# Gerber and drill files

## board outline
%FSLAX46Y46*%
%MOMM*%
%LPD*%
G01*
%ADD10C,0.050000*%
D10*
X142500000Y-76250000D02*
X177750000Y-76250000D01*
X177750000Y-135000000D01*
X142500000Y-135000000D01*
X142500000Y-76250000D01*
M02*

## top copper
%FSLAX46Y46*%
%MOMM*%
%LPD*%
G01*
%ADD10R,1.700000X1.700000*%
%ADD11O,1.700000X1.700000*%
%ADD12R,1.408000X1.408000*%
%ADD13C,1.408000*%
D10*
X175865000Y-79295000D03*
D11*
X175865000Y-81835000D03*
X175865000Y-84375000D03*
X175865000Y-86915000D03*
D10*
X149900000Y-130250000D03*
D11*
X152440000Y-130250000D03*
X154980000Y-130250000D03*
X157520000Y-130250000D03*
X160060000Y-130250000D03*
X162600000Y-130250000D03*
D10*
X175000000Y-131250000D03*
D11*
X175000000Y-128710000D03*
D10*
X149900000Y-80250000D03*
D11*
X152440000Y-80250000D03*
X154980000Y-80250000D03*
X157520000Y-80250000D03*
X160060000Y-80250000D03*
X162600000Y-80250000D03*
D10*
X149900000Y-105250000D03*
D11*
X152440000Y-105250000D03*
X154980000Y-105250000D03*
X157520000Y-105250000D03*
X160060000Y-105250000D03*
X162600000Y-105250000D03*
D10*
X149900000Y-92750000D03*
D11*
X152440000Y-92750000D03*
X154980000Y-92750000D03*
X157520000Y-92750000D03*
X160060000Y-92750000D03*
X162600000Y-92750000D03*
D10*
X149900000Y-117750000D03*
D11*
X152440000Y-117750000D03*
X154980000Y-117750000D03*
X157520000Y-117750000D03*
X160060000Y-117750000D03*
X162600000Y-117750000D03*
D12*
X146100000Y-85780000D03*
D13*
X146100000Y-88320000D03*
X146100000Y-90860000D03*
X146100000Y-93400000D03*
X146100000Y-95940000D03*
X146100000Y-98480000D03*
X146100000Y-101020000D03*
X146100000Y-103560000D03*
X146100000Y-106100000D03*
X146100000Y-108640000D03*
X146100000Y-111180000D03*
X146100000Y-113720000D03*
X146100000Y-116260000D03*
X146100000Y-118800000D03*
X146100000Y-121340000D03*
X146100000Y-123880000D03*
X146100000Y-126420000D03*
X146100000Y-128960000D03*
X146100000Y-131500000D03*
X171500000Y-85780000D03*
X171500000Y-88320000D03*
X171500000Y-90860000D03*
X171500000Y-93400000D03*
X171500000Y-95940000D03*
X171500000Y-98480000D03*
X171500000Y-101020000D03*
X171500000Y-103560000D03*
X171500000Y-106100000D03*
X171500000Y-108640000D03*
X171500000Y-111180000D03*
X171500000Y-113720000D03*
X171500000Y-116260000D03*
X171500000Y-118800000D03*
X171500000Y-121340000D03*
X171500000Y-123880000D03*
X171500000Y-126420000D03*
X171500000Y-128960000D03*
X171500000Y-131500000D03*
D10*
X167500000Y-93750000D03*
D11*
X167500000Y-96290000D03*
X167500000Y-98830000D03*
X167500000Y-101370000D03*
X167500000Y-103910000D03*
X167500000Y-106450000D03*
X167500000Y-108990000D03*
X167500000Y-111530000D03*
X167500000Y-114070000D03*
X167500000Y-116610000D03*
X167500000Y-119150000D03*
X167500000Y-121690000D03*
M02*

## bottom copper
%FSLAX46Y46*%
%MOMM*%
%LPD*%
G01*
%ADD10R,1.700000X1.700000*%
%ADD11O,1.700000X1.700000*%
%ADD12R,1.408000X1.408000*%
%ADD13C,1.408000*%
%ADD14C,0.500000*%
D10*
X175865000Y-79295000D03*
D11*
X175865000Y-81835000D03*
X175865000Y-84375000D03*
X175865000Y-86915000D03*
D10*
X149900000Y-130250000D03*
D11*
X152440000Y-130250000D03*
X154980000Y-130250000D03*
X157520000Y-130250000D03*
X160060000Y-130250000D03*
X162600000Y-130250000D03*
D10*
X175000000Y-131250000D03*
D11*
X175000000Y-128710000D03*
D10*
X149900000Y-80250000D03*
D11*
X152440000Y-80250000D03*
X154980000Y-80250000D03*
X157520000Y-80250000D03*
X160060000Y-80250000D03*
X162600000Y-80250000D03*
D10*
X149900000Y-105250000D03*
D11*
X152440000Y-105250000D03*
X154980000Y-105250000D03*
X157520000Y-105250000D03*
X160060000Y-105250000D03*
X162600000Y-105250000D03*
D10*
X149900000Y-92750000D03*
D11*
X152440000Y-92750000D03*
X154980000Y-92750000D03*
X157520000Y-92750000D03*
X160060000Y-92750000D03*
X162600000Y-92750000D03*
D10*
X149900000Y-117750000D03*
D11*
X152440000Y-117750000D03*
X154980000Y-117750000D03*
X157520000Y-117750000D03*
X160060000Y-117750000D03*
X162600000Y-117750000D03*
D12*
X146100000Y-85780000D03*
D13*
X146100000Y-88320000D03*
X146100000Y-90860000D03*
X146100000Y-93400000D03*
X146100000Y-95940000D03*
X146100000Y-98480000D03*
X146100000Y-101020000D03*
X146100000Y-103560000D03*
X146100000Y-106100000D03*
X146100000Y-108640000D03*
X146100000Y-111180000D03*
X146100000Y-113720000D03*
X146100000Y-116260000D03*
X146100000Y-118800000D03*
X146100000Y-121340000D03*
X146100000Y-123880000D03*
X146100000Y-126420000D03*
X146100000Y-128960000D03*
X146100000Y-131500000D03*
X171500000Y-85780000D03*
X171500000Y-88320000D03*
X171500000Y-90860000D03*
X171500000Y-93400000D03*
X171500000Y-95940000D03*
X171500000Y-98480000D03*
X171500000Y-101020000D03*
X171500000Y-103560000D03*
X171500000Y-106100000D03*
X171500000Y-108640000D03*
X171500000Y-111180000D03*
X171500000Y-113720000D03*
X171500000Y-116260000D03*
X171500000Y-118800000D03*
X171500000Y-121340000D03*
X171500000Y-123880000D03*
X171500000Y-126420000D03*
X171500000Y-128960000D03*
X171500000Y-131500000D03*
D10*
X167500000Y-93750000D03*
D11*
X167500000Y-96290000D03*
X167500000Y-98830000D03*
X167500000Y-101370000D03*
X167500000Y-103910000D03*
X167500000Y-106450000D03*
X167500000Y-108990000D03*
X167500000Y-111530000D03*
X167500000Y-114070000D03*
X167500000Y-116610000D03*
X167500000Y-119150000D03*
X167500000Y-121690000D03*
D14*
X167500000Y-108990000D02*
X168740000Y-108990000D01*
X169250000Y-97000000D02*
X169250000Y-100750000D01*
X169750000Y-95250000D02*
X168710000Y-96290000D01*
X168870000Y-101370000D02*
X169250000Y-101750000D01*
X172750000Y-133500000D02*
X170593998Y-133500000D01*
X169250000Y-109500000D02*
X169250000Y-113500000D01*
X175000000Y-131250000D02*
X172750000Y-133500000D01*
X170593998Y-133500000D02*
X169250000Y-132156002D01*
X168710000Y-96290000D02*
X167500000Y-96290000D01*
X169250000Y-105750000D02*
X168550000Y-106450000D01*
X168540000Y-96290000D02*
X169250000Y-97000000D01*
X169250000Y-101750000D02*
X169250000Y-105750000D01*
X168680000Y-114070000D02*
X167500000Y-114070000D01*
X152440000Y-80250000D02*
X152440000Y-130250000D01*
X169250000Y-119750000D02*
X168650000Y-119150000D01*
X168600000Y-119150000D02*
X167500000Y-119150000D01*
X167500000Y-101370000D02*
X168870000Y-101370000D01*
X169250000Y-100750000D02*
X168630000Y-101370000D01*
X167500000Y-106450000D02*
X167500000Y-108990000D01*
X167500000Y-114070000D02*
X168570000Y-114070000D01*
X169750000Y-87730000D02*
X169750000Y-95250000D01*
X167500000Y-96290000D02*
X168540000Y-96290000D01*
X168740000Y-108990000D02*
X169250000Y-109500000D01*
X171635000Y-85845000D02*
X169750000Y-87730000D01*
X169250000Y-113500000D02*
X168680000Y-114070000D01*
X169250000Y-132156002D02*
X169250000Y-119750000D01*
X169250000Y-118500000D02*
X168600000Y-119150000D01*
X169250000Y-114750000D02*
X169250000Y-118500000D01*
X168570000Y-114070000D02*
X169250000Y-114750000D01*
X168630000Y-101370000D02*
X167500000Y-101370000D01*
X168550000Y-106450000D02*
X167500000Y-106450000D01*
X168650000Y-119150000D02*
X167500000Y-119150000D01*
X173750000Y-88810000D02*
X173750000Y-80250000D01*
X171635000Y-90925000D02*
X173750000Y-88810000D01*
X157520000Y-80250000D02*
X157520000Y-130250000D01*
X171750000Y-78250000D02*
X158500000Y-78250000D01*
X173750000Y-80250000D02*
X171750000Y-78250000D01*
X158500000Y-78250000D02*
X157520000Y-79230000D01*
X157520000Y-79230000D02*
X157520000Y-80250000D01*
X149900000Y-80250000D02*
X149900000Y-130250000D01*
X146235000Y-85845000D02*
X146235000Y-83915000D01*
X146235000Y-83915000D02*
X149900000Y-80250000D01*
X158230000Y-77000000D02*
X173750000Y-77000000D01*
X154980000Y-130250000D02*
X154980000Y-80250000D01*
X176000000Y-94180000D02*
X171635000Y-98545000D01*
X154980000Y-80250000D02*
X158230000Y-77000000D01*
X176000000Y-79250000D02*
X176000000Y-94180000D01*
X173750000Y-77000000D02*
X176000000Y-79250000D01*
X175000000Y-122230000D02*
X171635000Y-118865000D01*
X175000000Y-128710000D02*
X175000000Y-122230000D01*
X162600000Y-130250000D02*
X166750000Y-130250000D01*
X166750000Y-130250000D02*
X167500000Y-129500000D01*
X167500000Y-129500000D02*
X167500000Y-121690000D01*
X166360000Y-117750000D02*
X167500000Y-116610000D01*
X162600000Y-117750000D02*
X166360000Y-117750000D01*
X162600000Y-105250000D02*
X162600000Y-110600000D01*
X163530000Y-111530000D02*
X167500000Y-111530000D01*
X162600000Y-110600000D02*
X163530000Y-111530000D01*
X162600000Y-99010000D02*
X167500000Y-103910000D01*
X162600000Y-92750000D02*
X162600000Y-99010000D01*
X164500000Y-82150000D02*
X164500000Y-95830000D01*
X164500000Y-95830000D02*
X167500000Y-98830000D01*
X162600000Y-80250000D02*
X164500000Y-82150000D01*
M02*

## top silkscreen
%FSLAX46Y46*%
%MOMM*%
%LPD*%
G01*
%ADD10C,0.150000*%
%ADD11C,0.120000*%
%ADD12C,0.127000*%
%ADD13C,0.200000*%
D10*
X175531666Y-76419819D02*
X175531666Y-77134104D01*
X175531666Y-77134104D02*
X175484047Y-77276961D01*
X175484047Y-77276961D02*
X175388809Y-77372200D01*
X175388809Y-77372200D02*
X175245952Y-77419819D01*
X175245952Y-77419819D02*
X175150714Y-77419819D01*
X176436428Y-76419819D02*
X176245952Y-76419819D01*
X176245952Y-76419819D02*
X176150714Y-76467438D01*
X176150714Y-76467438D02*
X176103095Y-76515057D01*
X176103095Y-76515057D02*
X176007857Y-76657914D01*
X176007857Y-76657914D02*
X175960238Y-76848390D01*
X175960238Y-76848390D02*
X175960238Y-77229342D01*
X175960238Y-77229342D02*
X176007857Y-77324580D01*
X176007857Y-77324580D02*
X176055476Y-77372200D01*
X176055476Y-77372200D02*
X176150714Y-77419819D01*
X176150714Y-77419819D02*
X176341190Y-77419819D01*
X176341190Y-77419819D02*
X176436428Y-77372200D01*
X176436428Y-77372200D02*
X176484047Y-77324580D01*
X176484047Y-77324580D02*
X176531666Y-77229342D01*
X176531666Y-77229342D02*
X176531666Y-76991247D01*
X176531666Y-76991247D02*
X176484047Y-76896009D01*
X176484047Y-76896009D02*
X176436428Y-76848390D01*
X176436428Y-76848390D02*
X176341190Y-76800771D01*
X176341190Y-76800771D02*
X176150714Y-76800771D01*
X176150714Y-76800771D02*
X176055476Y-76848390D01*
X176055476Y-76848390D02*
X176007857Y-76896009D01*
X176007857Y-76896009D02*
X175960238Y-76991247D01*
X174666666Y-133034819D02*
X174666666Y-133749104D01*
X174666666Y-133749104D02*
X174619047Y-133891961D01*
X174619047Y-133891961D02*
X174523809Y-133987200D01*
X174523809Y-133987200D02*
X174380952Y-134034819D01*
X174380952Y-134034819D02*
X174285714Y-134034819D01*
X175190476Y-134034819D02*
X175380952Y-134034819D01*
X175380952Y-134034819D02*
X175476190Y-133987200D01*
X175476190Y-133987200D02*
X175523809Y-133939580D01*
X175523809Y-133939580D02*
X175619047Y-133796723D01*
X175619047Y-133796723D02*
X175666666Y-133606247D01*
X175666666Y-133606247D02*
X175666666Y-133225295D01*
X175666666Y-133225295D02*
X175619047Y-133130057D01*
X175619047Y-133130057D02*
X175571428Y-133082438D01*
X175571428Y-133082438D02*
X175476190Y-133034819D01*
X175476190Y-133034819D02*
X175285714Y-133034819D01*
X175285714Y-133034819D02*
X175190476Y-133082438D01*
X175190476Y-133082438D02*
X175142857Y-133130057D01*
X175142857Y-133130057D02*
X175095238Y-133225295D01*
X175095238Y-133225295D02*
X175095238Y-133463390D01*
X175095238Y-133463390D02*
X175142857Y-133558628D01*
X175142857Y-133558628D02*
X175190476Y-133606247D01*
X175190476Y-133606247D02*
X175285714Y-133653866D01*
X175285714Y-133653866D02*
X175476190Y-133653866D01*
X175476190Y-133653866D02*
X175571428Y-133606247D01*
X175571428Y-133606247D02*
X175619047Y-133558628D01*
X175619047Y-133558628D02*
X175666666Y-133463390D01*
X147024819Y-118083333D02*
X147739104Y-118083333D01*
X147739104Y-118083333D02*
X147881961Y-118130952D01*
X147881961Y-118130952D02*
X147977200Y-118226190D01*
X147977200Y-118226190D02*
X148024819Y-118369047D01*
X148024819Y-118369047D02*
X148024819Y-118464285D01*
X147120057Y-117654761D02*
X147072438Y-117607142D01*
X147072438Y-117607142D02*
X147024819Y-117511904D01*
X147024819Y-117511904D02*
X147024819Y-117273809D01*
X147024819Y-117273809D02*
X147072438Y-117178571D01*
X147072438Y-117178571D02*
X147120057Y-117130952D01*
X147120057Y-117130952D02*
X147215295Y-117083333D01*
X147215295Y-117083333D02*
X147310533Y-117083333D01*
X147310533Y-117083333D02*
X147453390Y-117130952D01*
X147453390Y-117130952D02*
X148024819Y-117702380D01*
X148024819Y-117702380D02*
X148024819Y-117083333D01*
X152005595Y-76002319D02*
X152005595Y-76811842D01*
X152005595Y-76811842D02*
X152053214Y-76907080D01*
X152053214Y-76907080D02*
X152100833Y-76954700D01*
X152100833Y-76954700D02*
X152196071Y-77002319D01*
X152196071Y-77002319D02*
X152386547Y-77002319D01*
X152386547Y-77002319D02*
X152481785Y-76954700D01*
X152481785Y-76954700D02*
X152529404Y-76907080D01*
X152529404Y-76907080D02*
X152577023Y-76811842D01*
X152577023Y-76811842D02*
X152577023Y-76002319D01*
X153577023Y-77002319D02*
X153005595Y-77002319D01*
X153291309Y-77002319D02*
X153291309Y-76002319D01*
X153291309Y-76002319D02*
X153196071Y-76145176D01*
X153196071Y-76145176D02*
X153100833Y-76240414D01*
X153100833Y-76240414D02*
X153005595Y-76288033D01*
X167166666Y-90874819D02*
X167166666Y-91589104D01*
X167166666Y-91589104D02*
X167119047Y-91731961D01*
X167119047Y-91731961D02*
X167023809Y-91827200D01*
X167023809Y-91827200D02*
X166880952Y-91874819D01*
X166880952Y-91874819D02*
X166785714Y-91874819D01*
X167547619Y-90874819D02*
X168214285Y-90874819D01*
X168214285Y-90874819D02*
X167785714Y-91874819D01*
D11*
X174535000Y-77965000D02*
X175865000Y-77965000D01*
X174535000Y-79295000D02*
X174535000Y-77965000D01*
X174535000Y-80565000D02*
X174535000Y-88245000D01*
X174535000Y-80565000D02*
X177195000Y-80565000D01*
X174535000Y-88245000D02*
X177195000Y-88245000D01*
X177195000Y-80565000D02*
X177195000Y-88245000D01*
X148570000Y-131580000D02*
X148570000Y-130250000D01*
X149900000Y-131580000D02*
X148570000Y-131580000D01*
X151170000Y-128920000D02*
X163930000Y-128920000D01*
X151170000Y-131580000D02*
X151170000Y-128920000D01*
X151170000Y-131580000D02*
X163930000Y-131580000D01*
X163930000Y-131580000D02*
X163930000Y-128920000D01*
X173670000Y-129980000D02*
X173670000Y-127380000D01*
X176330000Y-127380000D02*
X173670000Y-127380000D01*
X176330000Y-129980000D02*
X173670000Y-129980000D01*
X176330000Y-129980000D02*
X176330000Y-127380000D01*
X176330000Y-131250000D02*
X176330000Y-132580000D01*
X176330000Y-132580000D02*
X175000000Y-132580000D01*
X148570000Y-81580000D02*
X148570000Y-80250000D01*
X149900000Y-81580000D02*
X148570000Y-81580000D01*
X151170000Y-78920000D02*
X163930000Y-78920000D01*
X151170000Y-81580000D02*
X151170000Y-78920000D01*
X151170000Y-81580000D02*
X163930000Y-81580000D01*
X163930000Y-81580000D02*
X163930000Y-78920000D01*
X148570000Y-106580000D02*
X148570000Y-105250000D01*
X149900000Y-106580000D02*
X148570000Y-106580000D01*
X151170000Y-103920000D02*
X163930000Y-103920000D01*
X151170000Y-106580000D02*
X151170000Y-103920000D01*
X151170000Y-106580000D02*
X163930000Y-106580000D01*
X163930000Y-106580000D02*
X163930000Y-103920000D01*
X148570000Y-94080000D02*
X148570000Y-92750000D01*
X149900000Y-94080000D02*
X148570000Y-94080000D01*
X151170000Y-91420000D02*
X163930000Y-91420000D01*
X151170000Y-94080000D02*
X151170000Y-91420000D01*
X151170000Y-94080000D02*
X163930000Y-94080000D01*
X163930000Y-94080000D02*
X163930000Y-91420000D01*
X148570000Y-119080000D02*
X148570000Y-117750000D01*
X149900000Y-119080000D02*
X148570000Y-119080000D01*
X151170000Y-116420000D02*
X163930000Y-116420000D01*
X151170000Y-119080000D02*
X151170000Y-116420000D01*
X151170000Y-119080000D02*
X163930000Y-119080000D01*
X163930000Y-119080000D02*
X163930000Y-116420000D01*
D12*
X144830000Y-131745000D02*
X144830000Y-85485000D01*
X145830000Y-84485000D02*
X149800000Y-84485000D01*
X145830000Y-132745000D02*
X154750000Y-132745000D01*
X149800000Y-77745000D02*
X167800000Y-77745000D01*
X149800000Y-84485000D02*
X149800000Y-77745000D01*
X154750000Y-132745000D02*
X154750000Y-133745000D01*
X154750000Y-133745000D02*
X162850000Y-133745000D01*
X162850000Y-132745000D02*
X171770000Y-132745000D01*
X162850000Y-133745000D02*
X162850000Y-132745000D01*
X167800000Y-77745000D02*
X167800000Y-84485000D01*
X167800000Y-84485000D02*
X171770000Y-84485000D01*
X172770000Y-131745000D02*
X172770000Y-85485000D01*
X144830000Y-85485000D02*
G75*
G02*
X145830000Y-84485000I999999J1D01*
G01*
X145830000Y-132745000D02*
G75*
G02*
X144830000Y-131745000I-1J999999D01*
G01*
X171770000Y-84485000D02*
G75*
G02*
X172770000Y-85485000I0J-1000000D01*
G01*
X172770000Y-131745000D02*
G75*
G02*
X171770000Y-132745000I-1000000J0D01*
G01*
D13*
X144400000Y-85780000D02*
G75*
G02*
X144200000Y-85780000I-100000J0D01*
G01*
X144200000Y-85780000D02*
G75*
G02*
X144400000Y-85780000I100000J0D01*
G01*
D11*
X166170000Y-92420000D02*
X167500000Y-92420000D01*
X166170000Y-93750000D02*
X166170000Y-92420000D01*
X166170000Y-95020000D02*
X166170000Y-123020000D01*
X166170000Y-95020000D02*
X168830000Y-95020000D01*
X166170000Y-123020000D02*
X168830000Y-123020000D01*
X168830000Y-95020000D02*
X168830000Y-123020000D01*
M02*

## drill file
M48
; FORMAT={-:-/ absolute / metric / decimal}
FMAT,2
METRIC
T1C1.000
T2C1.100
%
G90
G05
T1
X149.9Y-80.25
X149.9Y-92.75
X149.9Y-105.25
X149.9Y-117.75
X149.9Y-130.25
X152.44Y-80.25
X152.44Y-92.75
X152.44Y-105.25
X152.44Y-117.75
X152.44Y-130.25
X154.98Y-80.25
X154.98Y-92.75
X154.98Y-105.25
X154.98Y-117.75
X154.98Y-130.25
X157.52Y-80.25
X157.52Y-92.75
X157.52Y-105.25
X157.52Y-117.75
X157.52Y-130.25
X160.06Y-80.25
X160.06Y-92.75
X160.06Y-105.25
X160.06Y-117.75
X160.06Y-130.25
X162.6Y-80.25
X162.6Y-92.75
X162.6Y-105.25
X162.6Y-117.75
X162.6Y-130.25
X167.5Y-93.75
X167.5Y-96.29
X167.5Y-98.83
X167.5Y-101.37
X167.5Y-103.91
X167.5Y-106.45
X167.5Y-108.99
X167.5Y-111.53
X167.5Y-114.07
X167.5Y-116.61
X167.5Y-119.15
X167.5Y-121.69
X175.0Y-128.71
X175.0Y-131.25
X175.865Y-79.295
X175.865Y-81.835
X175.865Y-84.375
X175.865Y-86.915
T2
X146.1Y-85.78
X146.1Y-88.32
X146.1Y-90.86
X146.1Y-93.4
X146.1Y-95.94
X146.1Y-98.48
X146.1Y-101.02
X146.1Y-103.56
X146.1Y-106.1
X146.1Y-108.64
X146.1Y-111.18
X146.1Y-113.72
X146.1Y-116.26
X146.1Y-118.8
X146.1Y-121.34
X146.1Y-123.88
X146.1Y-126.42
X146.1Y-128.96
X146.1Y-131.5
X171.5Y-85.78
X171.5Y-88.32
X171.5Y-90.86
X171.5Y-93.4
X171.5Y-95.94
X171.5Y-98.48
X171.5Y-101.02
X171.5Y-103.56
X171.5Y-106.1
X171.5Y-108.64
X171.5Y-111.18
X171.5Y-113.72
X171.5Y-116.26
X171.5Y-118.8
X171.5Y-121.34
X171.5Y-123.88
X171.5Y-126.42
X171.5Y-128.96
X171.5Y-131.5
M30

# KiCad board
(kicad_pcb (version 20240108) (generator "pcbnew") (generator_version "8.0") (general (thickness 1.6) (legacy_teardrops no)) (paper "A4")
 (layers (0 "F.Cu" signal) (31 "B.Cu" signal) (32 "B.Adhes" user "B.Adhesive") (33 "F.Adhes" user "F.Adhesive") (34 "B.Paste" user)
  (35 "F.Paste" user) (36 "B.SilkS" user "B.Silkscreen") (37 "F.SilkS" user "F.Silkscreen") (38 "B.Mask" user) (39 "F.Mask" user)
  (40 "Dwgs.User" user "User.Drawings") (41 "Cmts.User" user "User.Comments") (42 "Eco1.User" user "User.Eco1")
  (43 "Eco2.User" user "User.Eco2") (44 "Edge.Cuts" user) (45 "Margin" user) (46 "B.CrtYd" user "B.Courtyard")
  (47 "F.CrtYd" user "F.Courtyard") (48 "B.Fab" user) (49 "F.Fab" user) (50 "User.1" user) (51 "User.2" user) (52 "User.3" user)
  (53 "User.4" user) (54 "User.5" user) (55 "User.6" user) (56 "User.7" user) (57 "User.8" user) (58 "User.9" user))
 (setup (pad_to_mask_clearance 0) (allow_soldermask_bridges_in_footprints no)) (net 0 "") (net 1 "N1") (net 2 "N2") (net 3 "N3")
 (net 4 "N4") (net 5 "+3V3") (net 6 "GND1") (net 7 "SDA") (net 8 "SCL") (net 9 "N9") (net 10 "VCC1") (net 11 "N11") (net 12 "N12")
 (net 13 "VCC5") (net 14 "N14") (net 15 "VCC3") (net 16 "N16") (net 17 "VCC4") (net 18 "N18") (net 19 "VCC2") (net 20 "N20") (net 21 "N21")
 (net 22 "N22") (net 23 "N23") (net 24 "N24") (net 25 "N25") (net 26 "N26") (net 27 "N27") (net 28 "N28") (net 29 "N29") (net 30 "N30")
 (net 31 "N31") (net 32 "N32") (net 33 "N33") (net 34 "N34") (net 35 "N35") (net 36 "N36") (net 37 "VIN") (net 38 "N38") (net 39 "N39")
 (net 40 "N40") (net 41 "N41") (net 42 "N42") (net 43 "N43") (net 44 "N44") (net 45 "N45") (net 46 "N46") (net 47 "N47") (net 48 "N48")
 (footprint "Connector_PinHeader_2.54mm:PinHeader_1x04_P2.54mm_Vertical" (layer "F.Cu") (at 175.865 79.295)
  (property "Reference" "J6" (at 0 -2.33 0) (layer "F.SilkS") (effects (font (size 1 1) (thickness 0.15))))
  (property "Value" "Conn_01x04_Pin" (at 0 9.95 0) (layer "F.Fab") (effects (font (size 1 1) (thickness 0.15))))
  (fp_line (start -1.33 -1.33) (end 0 -1.33) (stroke (width 0.12) (type solid)) (layer "F.SilkS"))
  (fp_line (start -1.33 0) (end -1.33 -1.33) (stroke (width 0.12) (type solid)) (layer "F.SilkS"))
  (fp_line (start -1.33 1.27) (end -1.33 8.95) (stroke (width 0.12) (type solid)) (layer "F.SilkS"))
  (fp_line (start -1.33 1.27) (end 1.33 1.27) (stroke (width 0.12) (type solid)) (layer "F.SilkS"))
  (fp_line (start -1.33 8.95) (end 1.33 8.95) (stroke (width 0.12) (type solid)) (layer "F.SilkS"))
  (fp_line (start 1.33 1.27) (end 1.33 8.95) (stroke (width 0.12) (type solid)) (layer "F.SilkS"))
  (pad "1" thru_hole rect (at 0 0) (size 1.7 1.7) (drill 1) (layers "*.Cu" "*.Mask") (remove_unused_layers no) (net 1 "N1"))
  (pad "2" thru_hole oval (at 0 2.54) (size 1.7 1.7) (drill 1) (layers "*.Cu" "*.Mask") (remove_unused_layers no) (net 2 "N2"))
  (pad "3" thru_hole oval (at 0 5.08) (size 1.7 1.7) (drill 1) (layers "*.Cu" "*.Mask") (remove_unused_layers no) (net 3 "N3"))
  (pad "4" thru_hole oval (at 0 7.62) (size 1.7 1.7) (drill 1) (layers "*.Cu" "*.Mask") (remove_unused_layers no) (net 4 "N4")))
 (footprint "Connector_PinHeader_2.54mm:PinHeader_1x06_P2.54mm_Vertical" (layer "F.Cu") (at 149.9 130.25 90)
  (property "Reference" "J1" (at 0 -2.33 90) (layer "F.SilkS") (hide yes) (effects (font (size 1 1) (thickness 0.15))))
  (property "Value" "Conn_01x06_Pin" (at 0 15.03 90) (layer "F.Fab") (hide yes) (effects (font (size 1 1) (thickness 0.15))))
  (fp_line (start -1.33 -1.33) (end 0 -1.33) (stroke (width 0.12) (type solid)) (layer "F.SilkS"))
  (fp_line (start -1.33 0) (end -1.33 -1.33) (stroke (width 0.12) (type solid)) (layer "F.SilkS"))
  (fp_line (start 1.33 1.27) (end 1.33 14.03) (stroke (width 0.12) (type solid)) (layer "F.SilkS"))
  (fp_line (start -1.33 1.27) (end 1.33 1.27) (stroke (width 0.12) (type solid)) (layer "F.SilkS"))
  (fp_line (start -1.33 1.27) (end -1.33 14.03) (stroke (width 0.12) (type solid)) (layer "F.SilkS"))
  (fp_line (start -1.33 14.03) (end 1.33 14.03) (stroke (width 0.12) (type solid)) (layer "F.SilkS"))
  (pad "1" thru_hole rect (at 0 0 90) (size 1.7 1.7) (drill 1) (layers "*.Cu" "*.Mask") (remove_unused_layers no) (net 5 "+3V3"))
  (pad "2" thru_hole oval (at 0 2.54 90) (size 1.7 1.7) (drill 1) (layers "*.Cu" "*.Mask") (remove_unused_layers no) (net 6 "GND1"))
  (pad "3" thru_hole oval (at 0 5.08 90) (size 1.7 1.7) (drill 1) (layers "*.Cu" "*.Mask") (remove_unused_layers no) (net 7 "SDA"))
  (pad "4" thru_hole oval (at 0 7.62 90) (size 1.7 1.7) (drill 1) (layers "*.Cu" "*.Mask") (remove_unused_layers no) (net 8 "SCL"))
  (pad "5" thru_hole oval (at 0 10.16 90) (size 1.7 1.7) (drill 1) (layers "*.Cu" "*.Mask") (remove_unused_layers no) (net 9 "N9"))
  (pad "6" thru_hole oval (at 0 12.7 90) (size 1.7 1.7) (drill 1) (layers "*.Cu" "*.Mask") (remove_unused_layers no) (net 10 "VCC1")))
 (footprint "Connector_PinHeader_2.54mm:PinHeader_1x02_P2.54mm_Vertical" (layer "F.Cu") (at 175 131.25 180)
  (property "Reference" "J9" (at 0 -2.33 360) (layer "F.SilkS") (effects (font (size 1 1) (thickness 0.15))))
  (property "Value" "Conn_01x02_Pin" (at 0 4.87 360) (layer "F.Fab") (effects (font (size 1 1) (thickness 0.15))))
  (fp_line (start 1.33 1.27) (end 1.33 3.87) (stroke (width 0.12) (type solid)) (layer "F.SilkS"))
  (fp_line (start -1.33 3.87) (end 1.33 3.87) (stroke (width 0.12) (type solid)) (layer "F.SilkS"))
  (fp_line (start -1.33 1.27) (end 1.33 1.27) (stroke (width 0.12) (type solid)) (layer "F.SilkS"))
  (fp_line (start -1.33 1.27) (end -1.33 3.87) (stroke (width 0.12) (type solid)) (layer "F.SilkS"))
  (fp_line (start -1.33 0) (end -1.33 -1.33) (stroke (width 0.12) (type solid)) (layer "F.SilkS"))
  (fp_line (start -1.33 -1.33) (end 0 -1.33) (stroke (width 0.12) (type solid)) (layer "F.SilkS"))
  (pad "1" thru_hole rect (at 0 0 180) (size 1.7 1.7) (drill 1) (layers "*.Cu" "*.Mask") (remove_unused_layers no) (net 6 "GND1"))
  (pad "2" thru_hole oval (at 0 2.54 180) (size 1.7 1.7) (drill 1) (layers "*.Cu" "*.Mask") (remove_unused_layers no) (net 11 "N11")))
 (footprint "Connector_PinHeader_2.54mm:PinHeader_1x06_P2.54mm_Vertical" (layer "F.Cu") (at 149.9 80.25 90)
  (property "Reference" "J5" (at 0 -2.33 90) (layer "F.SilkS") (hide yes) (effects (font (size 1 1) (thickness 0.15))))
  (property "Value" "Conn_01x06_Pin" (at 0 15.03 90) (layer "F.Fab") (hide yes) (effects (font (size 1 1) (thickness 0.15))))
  (fp_line (start -1.33 -1.33) (end 0 -1.33) (stroke (width 0.12) (type solid)) (layer "F.SilkS"))
  (fp_line (start -1.33 0) (end -1.33 -1.33) (stroke (width 0.12) (type solid)) (layer "F.SilkS"))
  (fp_line (start 1.33 1.27) (end 1.33 14.03) (stroke (width 0.12) (type solid)) (layer "F.SilkS"))
  (fp_line (start -1.33 1.27) (end 1.33 1.27) (stroke (width 0.12) (type solid)) (layer "F.SilkS"))
  (fp_line (start -1.33 1.27) (end -1.33 14.03) (stroke (width 0.12) (type solid)) (layer "F.SilkS"))
  (fp_line (start -1.33 14.03) (end 1.33 14.03) (stroke (width 0.12) (type solid)) (layer "F.SilkS"))
  (pad "1" thru_hole rect (at 0 0 90) (size 1.7 1.7) (drill 1) (layers "*.Cu" "*.Mask") (remove_unused_layers no) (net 5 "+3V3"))
  (pad "2" thru_hole oval (at 0 2.54 90) (size 1.7 1.7) (drill 1) (layers "*.Cu" "*.Mask") (remove_unused_layers no) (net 6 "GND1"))
  (pad "3" thru_hole oval (at 0 5.08 90) (size 1.7 1.7) (drill 1) (layers "*.Cu" "*.Mask") (remove_unused_layers no) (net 7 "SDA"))
  (pad "4" thru_hole oval (at 0 7.62 90) (size 1.7 1.7) (drill 1) (layers "*.Cu" "*.Mask") (remove_unused_layers no) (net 8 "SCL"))
  (pad "5" thru_hole oval (at 0 10.16 90) (size 1.7 1.7) (drill 1) (layers "*.Cu" "*.Mask") (remove_unused_layers no) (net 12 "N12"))
  (pad "6" thru_hole oval (at 0 12.7 90) (size 1.7 1.7) (drill 1) (layers "*.Cu" "*.Mask") (remove_unused_layers no) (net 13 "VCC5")))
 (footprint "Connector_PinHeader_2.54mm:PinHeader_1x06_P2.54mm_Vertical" (layer "F.Cu") (at 149.9 105.25 90)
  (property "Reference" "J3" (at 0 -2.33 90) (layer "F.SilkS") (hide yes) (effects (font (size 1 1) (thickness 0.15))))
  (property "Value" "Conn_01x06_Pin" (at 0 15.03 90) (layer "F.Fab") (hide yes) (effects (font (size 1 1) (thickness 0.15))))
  (fp_line (start -1.33 -1.33) (end 0 -1.33) (stroke (width 0.12) (type solid)) (layer "F.SilkS"))
  (fp_line (start -1.33 0) (end -1.33 -1.33) (stroke (width 0.12) (type solid)) (layer "F.SilkS"))
  (fp_line (start 1.33 1.27) (end 1.33 14.03) (stroke (width 0.12) (type solid)) (layer "F.SilkS"))
  (fp_line (start -1.33 1.27) (end 1.33 1.27) (stroke (width 0.12) (type solid)) (layer "F.SilkS"))
  (fp_line (start -1.33 1.27) (end -1.33 14.03) (stroke (width 0.12) (type solid)) (layer "F.SilkS"))
  (fp_line (start -1.33 14.03) (end 1.33 14.03) (stroke (width 0.12) (type solid)) (layer "F.SilkS"))
  (pad "1" thru_hole rect (at 0 0 90) (size 1.7 1.7) (drill 1) (layers "*.Cu" "*.Mask") (remove_unused_layers no) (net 5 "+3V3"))
  (pad "2" thru_hole oval (at 0 2.54 90) (size 1.7 1.7) (drill 1) (layers "*.Cu" "*.Mask") (remove_unused_layers no) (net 6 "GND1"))
  (pad "3" thru_hole oval (at 0 5.08 90) (size 1.7 1.7) (drill 1) (layers "*.Cu" "*.Mask") (remove_unused_layers no) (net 7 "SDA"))
  (pad "4" thru_hole oval (at 0 7.62 90) (size 1.7 1.7) (drill 1) (layers "*.Cu" "*.Mask") (remove_unused_layers no) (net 8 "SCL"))
  (pad "5" thru_hole oval (at 0 10.16 90) (size 1.7 1.7) (drill 1) (layers "*.Cu" "*.Mask") (remove_unused_layers no) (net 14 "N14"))
  (pad "6" thru_hole oval (at 0 12.7 90) (size 1.7 1.7) (drill 1) (layers "*.Cu" "*.Mask") (remove_unused_layers no) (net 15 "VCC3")))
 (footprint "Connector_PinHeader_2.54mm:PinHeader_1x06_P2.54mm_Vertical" (layer "F.Cu") (at 149.9 92.75 90)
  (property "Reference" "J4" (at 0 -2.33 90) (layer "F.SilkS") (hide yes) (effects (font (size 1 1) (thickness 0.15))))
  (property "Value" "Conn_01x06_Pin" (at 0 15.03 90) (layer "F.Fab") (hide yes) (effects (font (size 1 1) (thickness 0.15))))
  (fp_line (start -1.33 -1.33) (end 0 -1.33) (stroke (width 0.12) (type solid)) (layer "F.SilkS"))
  (fp_line (start -1.33 0) (end -1.33 -1.33) (stroke (width 0.12) (type solid)) (layer "F.SilkS"))
  (fp_line (start 1.33 1.27) (end 1.33 14.03) (stroke (width 0.12) (type solid)) (layer "F.SilkS"))
  (fp_line (start -1.33 1.27) (end 1.33 1.27) (stroke (width 0.12) (type solid)) (layer "F.SilkS"))
  (fp_line (start -1.33 1.27) (end -1.33 14.03) (stroke (width 0.12) (type solid)) (layer "F.SilkS"))
  (fp_line (start -1.33 14.03) (end 1.33 14.03) (stroke (width 0.12) (type solid)) (layer "F.SilkS"))
  (pad "1" thru_hole rect (at 0 0 90) (size 1.7 1.7) (drill 1) (layers "*.Cu" "*.Mask") (remove_unused_layers no) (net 5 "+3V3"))
  (pad "2" thru_hole oval (at 0 2.54 90) (size 1.7 1.7) (drill 1) (layers "*.Cu" "*.Mask") (remove_unused_layers no) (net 6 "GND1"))
  (pad "3" thru_hole oval (at 0 5.08 90) (size 1.7 1.7) (drill 1) (layers "*.Cu" "*.Mask") (remove_unused_layers no) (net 7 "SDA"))
  (pad "4" thru_hole oval (at 0 7.62 90) (size 1.7 1.7) (drill 1) (layers "*.Cu" "*.Mask") (remove_unused_layers no) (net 8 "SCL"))
  (pad "5" thru_hole oval (at 0 10.16 90) (size 1.7 1.7) (drill 1) (layers "*.Cu" "*.Mask") (remove_unused_layers no) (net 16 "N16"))
  (pad "6" thru_hole oval (at 0 12.7 90) (size 1.7 1.7) (drill 1) (layers "*.Cu" "*.Mask") (remove_unused_layers no) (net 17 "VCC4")))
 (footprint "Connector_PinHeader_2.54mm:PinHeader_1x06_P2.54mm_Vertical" (layer "F.Cu") (at 149.9 117.75 90)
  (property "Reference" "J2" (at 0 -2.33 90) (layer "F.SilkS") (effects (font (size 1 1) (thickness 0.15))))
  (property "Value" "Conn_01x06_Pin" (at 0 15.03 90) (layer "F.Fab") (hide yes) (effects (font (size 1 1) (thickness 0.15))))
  (fp_line (start -1.33 -1.33) (end 0 -1.33) (stroke (width 0.12) (type solid)) (layer "F.SilkS"))
  (fp_line (start -1.33 0) (end -1.33 -1.33) (stroke (width 0.12) (type solid)) (layer "F.SilkS"))
  (fp_line (start 1.33 1.27) (end 1.33 14.03) (stroke (width 0.12) (type solid)) (layer "F.SilkS"))
  (fp_line (start -1.33 1.27) (end 1.33 1.27) (stroke (width 0.12) (type solid)) (layer "F.SilkS"))
  (fp_line (start -1.33 1.27) (end -1.33 14.03) (stroke (width 0.12) (type solid)) (layer "F.SilkS"))
  (fp_line (start -1.33 14.03) (end 1.33 14.03) (stroke (width 0.12) (type solid)) (layer "F.SilkS"))
  (pad "1" thru_hole rect (at 0 0 90) (size 1.7 1.7) (drill 1) (layers "*.Cu" "*.Mask") (remove_unused_layers no) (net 5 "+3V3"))
  (pad "2" thru_hole oval (at 0 2.54 90) (size 1.7 1.7) (drill 1) (layers "*.Cu" "*.Mask") (remove_unused_layers no) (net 6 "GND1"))
  (pad "3" thru_hole oval (at 0 5.08 90) (size 1.7 1.7) (drill 1) (layers "*.Cu" "*.Mask") (remove_unused_layers no) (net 7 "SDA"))
  (pad "4" thru_hole oval (at 0 7.62 90) (size 1.7 1.7) (drill 1) (layers "*.Cu" "*.Mask") (remove_unused_layers no) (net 8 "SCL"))
  (pad "5" thru_hole oval (at 0 10.16 90) (size 1.7 1.7) (drill 1) (layers "*.Cu" "*.Mask") (remove_unused_layers no) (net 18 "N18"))
  (pad "6" thru_hole oval (at 0 12.7 90) (size 1.7 1.7) (drill 1) (layers "*.Cu" "*.Mask") (remove_unused_layers no) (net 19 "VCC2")))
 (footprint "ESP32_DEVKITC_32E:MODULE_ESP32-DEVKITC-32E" (layer "F.Cu") (at 158.8 108.615)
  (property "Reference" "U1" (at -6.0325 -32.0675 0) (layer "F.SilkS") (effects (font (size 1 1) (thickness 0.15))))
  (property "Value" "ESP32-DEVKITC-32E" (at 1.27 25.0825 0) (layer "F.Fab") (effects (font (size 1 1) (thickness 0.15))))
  (fp_line (start -13.97 23.13) (end -13.97 -23.13) (stroke (width 0.127) (type solid)) (layer "F.SilkS"))
  (fp_line (start -12.97 -24.13) (end -9 -24.13) (stroke (width 0.127) (type solid)) (layer "F.SilkS"))
  (fp_line (start -12.97 24.13) (end -4.05 24.13) (stroke (width 0.127) (type solid)) (layer "F.SilkS"))
  (fp_line (start -9 -30.87) (end 9 -30.87) (stroke (width 0.127) (type solid)) (layer "F.SilkS"))
  (fp_line (start -9 -24.13) (end -9 -30.87) (stroke (width 0.127) (type solid)) (layer "F.SilkS"))
  (fp_line (start -4.05 24.13) (end -4.05 25.13) (stroke (width 0.127) (type solid)) (layer "F.SilkS"))
  (fp_line (start -4.05 25.13) (end 4.05 25.13) (stroke (width 0.127) (type solid)) (layer "F.SilkS"))
  (fp_line (start 4.05 24.13) (end 12.97 24.13) (stroke (width 0.127) (type solid)) (layer "F.SilkS"))
  (fp_line (start 4.05 25.13) (end 4.05 24.13) (stroke (width 0.127) (type solid)) (layer "F.SilkS"))
  (fp_line (start 9 -30.87) (end 9 -24.13) (stroke (width 0.127) (type solid)) (layer "F.SilkS"))
  (fp_line (start 9 -24.13) (end 12.97 -24.13) (stroke (width 0.127) (type solid)) (layer "F.SilkS"))
  (fp_line (start 13.97 23.13) (end 13.97 -23.13) (stroke (width 0.127) (type solid)) (layer "F.SilkS"))
  (fp_arc (start -13.97 -23.13) (mid -13.677107 -23.837107) (end -12.97 -24.13) (stroke (width 0.127) (type solid)) (layer "F.SilkS"))
  (fp_arc (start -12.97 24.13) (mid -13.677107 23.837107) (end -13.97 23.13) (stroke (width 0.127) (type solid)) (layer "F.SilkS"))
  (fp_arc (start 12.97 -24.13) (mid 13.677107 -23.837107) (end 13.97 -23.13) (stroke (width 0.127) (type solid)) (layer "F.SilkS"))
  (fp_arc (start 13.97 23.13) (mid 13.677107 23.837107) (end 12.97 24.13) (stroke (width 0.127) (type solid)) (layer "F.SilkS"))
  (fp_circle (center -14.5 -22.835) (end -14.4 -22.835) (stroke (width 0.2) (type solid)) (fill none) (layer "F.SilkS"))
  (pad "J2_1" thru_hole rect (at -12.7 -22.835) (size 1.408 1.408) (drill 1.1) (layers "*.Cu" "*.Mask") (remove_unused_layers no)
   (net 5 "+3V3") (solder_mask_margin 0.102))
  (pad "J2_2" thru_hole circle (at -12.7 -20.295) (size 1.408 1.408) (drill 1.1) (layers "*.Cu" "*.Mask") (remove_unused_layers no)
   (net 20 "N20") (solder_mask_margin 0.102))
  (pad "J2_3" thru_hole circle (at -12.7 -17.755) (size 1.408 1.408) (drill 1.1) (layers "*.Cu" "*.Mask") (remove_unused_layers no)
   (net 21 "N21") (solder_mask_margin 0.102))
  (pad "J2_4" thru_hole circle (at -12.7 -15.215) (size 1.408 1.408) (drill 1.1) (layers "*.Cu" "*.Mask") (remove_unused_layers no)
   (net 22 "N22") (solder_mask_margin 0.102))
  (pad "J2_5" thru_hole circle (at -12.7 -12.675) (size 1.408 1.408) (drill 1.1) (layers "*.Cu" "*.Mask") (remove_unused_layers no)
   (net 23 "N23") (solder_mask_margin 0.102))
  (pad "J2_6" thru_hole circle (at -12.7 -10.135) (size 1.408 1.408) (drill 1.1) (layers "*.Cu" "*.Mask") (remove_unused_layers no)
   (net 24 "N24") (solder_mask_margin 0.102))
  (pad "J2_7" thru_hole circle (at -12.7 -7.595) (size 1.408 1.408) (drill 1.1) (layers "*.Cu" "*.Mask") (remove_unused_layers no)
   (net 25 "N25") (solder_mask_margin 0.102))
  (pad "J2_8" thru_hole circle (at -12.7 -5.055) (size 1.408 1.408) (drill 1.1) (layers "*.Cu" "*.Mask") (remove_unused_layers no)
   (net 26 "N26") (solder_mask_margin 0.102))
  (pad "J2_9" thru_hole circle (at -12.7 -2.515) (size 1.408 1.408) (drill 1.1) (layers "*.Cu" "*.Mask") (remove_unused_layers no)
   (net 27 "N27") (solder_mask_margin 0.102))
  (pad "J2_10" thru_hole circle (at -12.7 0.025) (size 1.408 1.408) (drill 1.1) (layers "*.Cu" "*.Mask") (remove_unused_layers no)
   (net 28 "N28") (solder_mask_margin 0.102))
  (pad "J2_11" thru_hole circle (at -12.7 2.565) (size 1.408 1.408) (drill 1.1) (layers "*.Cu" "*.Mask") (remove_unused_layers no)
   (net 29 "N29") (solder_mask_margin 0.102))
  (pad "J2_12" thru_hole circle (at -12.7 5.105) (size 1.408 1.408) (drill 1.1) (layers "*.Cu" "*.Mask") (remove_unused_layers no)
   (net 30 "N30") (solder_mask_margin 0.102))
  (pad "J2_13" thru_hole circle (at -12.7 7.645) (size 1.408 1.408) (drill 1.1) (layers "*.Cu" "*.Mask") (remove_unused_layers no)
   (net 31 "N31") (solder_mask_margin 0.102))
  (pad "J2_14" thru_hole circle (at -12.7 10.185) (size 1.408 1.408) (drill 1.1) (layers "*.Cu" "*.Mask") (remove_unused_layers no)
   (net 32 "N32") (solder_mask_margin 0.102))
  (pad "J2_15" thru_hole circle (at -12.7 12.725) (size 1.408 1.408) (drill 1.1) (layers "*.Cu" "*.Mask") (remove_unused_layers no)
   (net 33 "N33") (solder_mask_margin 0.102))
  (pad "J2_16" thru_hole circle (at -12.7 15.265) (size 1.408 1.408) (drill 1.1) (layers "*.Cu" "*.Mask") (remove_unused_layers no)
   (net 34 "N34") (solder_mask_margin 0.102))
  (pad "J2_17" thru_hole circle (at -12.7 17.805) (size 1.408 1.408) (drill 1.1) (layers "*.Cu" "*.Mask") (remove_unused_layers no)
   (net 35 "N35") (solder_mask_margin 0.102))
  (pad "J2_18" thru_hole circle (at -12.7 20.345) (size 1.408 1.408) (drill 1.1) (layers "*.Cu" "*.Mask") (remove_unused_layers no)
   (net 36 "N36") (solder_mask_margin 0.102))
  (pad "J2_19" thru_hole circle (at -12.7 22.885) (size 1.408 1.408) (drill 1.1) (layers "*.Cu" "*.Mask") (remove_unused_layers no)
   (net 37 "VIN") (solder_mask_margin 0.102))
  (pad "J3_1" thru_hole circle (at 12.7 -22.835) (size 1.408 1.408) (drill 1.1) (layers "*.Cu" "*.Mask") (remove_unused_layers no)
   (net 6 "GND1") (solder_mask_margin 0.102))
  (pad "J3_2" thru_hole circle (at 12.7 -20.295) (size 1.408 1.408) (drill 1.1) (layers "*.Cu" "*.Mask") (remove_unused_layers no)
   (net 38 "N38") (solder_mask_margin 0.102))
  (pad "J3_3" thru_hole circle (at 12.7 -17.755) (size 1.408 1.408) (drill 1.1) (layers "*.Cu" "*.Mask") (remove_unused_layers no)
   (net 8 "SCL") (solder_mask_margin 0.102))
  (pad "J3_4" thru_hole circle (at 12.7 -15.215) (size 1.408 1.408) (drill 1.1) (layers "*.Cu" "*.Mask") (remove_unused_layers no)
   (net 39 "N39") (solder_mask_margin 0.102))
  (pad "J3_5" thru_hole circle (at 12.7 -12.675) (size 1.408 1.408) (drill 1.1) (layers "*.Cu" "*.Mask") (remove_unused_layers no)
   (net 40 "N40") (solder_mask_margin 0.102))
  (pad "J3_6" thru_hole circle (at 12.7 -10.135) (size 1.408 1.408) (drill 1.1) (layers "*.Cu" "*.Mask") (remove_unused_layers no)
   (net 7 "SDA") (solder_mask_margin 0.102))
  (pad "J3_7" thru_hole circle (at 12.7 -7.595) (size 1.408 1.408) (drill 1.1) (layers "*.Cu" "*.Mask") (remove_unused_layers no)
   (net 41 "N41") (solder_mask_margin 0.102))
  (pad "J3_8" thru_hole circle (at 12.7 -5.055) (size 1.408 1.408) (drill 1.1) (layers "*.Cu" "*.Mask") (remove_unused_layers no)
   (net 4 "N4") (solder_mask_margin 0.102))
  (pad "J3_9" thru_hole circle (at 12.7 -2.515) (size 1.408 1.408) (drill 1.1) (layers "*.Cu" "*.Mask") (remove_unused_layers no)
   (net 3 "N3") (solder_mask_margin 0.102))
  (pad "J3_10" thru_hole circle (at 12.7 0.025) (size 1.408 1.408) (drill 1.1) (layers "*.Cu" "*.Mask") (remove_unused_layers no)
   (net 2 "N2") (solder_mask_margin 0.102))
  (pad "J3_11" thru_hole circle (at 12.7 2.565) (size 1.408 1.408) (drill 1.1) (layers "*.Cu" "*.Mask") (remove_unused_layers no)
   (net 1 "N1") (solder_mask_margin 0.102))
  (pad "J3_12" thru_hole circle (at 12.7 5.105) (size 1.408 1.408) (drill 1.1) (layers "*.Cu" "*.Mask") (remove_unused_layers no)
   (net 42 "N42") (solder_mask_margin 0.102))
  (pad "J3_13" thru_hole circle (at 12.7 7.645) (size 1.408 1.408) (drill 1.1) (layers "*.Cu" "*.Mask") (remove_unused_layers no)
   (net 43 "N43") (solder_mask_margin 0.102))
  (pad "J3_14" thru_hole circle (at 12.7 10.185) (size 1.408 1.408) (drill 1.1) (layers "*.Cu" "*.Mask") (remove_unused_layers no)
   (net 11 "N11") (solder_mask_margin 0.102))
  (pad "J3_15" thru_hole circle (at 12.7 12.725) (size 1.408 1.408) (drill 1.1) (layers "*.Cu" "*.Mask") (remove_unused_layers no)
   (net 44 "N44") (solder_mask_margin 0.102))
  (pad "J3_16" thru_hole circle (at 12.7 15.265) (size 1.408 1.408) (drill 1.1) (layers "*.Cu" "*.Mask") (remove_unused_layers no)
   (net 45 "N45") (solder_mask_margin 0.102))
  (pad "J3_17" thru_hole circle (at 12.7 17.805) (size 1.408 1.408) (drill 1.1) (layers "*.Cu" "*.Mask") (remove_unused_layers no)
   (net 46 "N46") (solder_mask_margin 0.102))
  (pad "J3_18" thru_hole circle (at 12.7 20.345) (size 1.408 1.408) (drill 1.1) (layers "*.Cu" "*.Mask") (remove_unused_layers no)
   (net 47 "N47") (solder_mask_margin 0.102))
  (pad "J3_19" thru_hole circle (at 12.7 22.885) (size 1.408 1.408) (drill 1.1) (layers "*.Cu" "*.Mask") (remove_unused_layers no)
   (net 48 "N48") (solder_mask_margin 0.102)))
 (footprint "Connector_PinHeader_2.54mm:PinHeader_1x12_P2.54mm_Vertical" (layer "F.Cu") (at 167.5 93.75)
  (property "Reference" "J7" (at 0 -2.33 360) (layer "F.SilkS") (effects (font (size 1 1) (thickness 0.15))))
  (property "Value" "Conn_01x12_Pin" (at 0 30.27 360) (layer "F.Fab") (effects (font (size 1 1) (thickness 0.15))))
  (fp_line (start -1.33 -1.33) (end 0 -1.33) (stroke (width 0.12) (type solid)) (layer "F.SilkS"))
  (fp_line (start -1.33 0) (end -1.33 -1.33) (stroke (width 0.12) (type solid)) (layer "F.SilkS"))
  (fp_line (start -1.33 1.27) (end -1.33 29.27) (stroke (width 0.12) (type solid)) (layer "F.SilkS"))
  (fp_line (start -1.33 1.27) (end 1.33 1.27) (stroke (width 0.12) (type solid)) (layer "F.SilkS"))
  (fp_line (start -1.33 29.27) (end 1.33 29.27) (stroke (width 0.12) (type solid)) (layer "F.SilkS"))
  (fp_line (start 1.33 1.27) (end 1.33 29.27) (stroke (width 0.12) (type solid)) (layer "F.SilkS"))
  (pad "1" thru_hole rect (at 0 0) (size 1.7 1.7) (drill 1) (layers "*.Cu" "*.Mask") (remove_unused_layers no) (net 37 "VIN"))
  (pad "2" thru_hole oval (at 0 2.54) (size 1.7 1.7) (drill 1) (layers "*.Cu" "*.Mask") (remove_unused_layers no) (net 6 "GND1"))
  (pad "3" thru_hole oval (at 0 5.08) (size 1.7 1.7) (drill 1) (layers "*.Cu" "*.Mask") (remove_unused_layers no) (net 13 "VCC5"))
  (pad "4" thru_hole oval (at 0 7.62) (size 1.7 1.7) (drill 1) (layers "*.Cu" "*.Mask") (remove_unused_layers no) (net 6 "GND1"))
  (pad "5" thru_hole oval (at 0 10.16) (size 1.7 1.7) (drill 1) (layers "*.Cu" "*.Mask") (remove_unused_layers no) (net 17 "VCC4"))
  (pad "6" thru_hole oval (at 0 12.7) (size 1.7 1.7) (drill 1) (layers "*.Cu" "*.Mask") (remove_unused_layers no) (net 6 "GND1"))
  (pad "7" thru_hole oval (at 0 15.24) (size 1.7 1.7) (drill 1) (layers "*.Cu" "*.Mask") (remove_unused_layers no) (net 6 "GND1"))
  (pad "8" thru_hole oval (at 0 17.78) (size 1.7 1.7) (drill 1) (layers "*.Cu" "*.Mask") (remove_unused_layers no) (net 15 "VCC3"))
  (pad "9" thru_hole oval (at 0 20.32) (size 1.7 1.7) (drill 1) (layers "*.Cu" "*.Mask") (remove_unused_layers no) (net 6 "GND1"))
  (pad "10" thru_hole oval (at 0 22.86) (size 1.7 1.7) (drill 1) (layers "*.Cu" "*.Mask") (remove_unused_layers no) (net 19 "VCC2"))
  (pad "11" thru_hole oval (at 0 25.4) (size 1.7 1.7) (drill 1) (layers "*.Cu" "*.Mask") (remove_unused_layers no) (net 6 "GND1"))
  (pad "12" thru_hole oval (at 0 27.94) (size 1.7 1.7) (drill 1) (layers "*.Cu" "*.Mask") (remove_unused_layers no) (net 10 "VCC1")))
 (gr_rect (start 142.5 76.25) (end 177.75 135) (stroke (width 0.05) (type default)) (fill none) (layer "Edge.Cuts"))
 (segment (start 167.5 108.99) (end 168.74 108.99) (width 0.5) (layer "B.Cu") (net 6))
 (segment (start 169.25 97) (end 169.25 100.75) (width 0.5) (layer "B.Cu") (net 6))
 (segment (start 169.75 95.25) (end 168.71 96.29) (width 0.5) (layer "B.Cu") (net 6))
 (segment (start 168.87 101.37) (end 169.25 101.75) (width 0.5) (layer "B.Cu") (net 6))
 (segment (start 172.75 133.5) (end 170.593998 133.5) (width 0.5) (layer "B.Cu") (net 6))
 (segment (start 169.25 109.5) (end 169.25 113.5) (width 0.5) (layer "B.Cu") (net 6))
 (segment (start 175 131.25) (end 172.75 133.5) (width 0.5) (layer "B.Cu") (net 6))
 (segment (start 170.593998 133.5) (end 169.25 132.156002) (width 0.5) (layer "B.Cu") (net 6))
 (segment (start 168.71 96.29) (end 167.5 96.29) (width 0.5) (layer "B.Cu") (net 6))
 (segment (start 169.25 105.75) (end 168.55 106.45) (width 0.5) (layer "B.Cu") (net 6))
 (segment (start 168.54 96.29) (end 169.25 97) (width 0.5) (layer "B.Cu") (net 6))
 (segment (start 169.25 101.75) (end 169.25 105.75) (width 0.5) (layer "B.Cu") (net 6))
 (segment (start 168.68 114.07) (end 167.5 114.07) (width 0.5) (layer "B.Cu") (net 6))
 (segment (start 152.44 80.25) (end 152.44 130.25) (width 0.5) (layer "B.Cu") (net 6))
 (segment (start 169.25 119.75) (end 168.65 119.15) (width 0.5) (layer "B.Cu") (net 6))
 (segment (start 168.6 119.15) (end 167.5 119.15) (width 0.5) (layer "B.Cu") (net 6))
 (segment (start 167.5 101.37) (end 168.87 101.37) (width 0.5) (layer "B.Cu") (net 6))
 (segment (start 169.25 100.75) (end 168.63 101.37) (width 0.5) (layer "B.Cu") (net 6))
 (segment (start 167.5 106.45) (end 167.5 108.99) (width 0.5) (layer "B.Cu") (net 6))
 (segment (start 167.5 114.07) (end 168.57 114.07) (width 0.5) (layer "B.Cu") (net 6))
 (segment (start 169.75 87.73) (end 169.75 95.25) (width 0.5) (layer "B.Cu") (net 6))
 (segment (start 167.5 96.29) (end 168.54 96.29) (width 0.5) (layer "B.Cu") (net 6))
 (segment (start 168.74 108.99) (end 169.25 109.5) (width 0.5) (layer "B.Cu") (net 6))
 (segment (start 171.635 85.845) (end 169.75 87.73) (width 0.5) (layer "B.Cu") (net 6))
 (segment (start 169.25 113.5) (end 168.68 114.07) (width 0.5) (layer "B.Cu") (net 6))
 (segment (start 169.25 132.156002) (end 169.25 119.75) (width 0.5) (layer "B.Cu") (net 6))
 (segment (start 169.25 118.5) (end 168.6 119.15) (width 0.5) (layer "B.Cu") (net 6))
 (segment (start 169.25 114.75) (end 169.25 118.5) (width 0.5) (layer "B.Cu") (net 6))
 (segment (start 168.57 114.07) (end 169.25 114.75) (width 0.5) (layer "B.Cu") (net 6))
 (segment (start 168.63 101.37) (end 167.5 101.37) (width 0.5) (layer "B.Cu") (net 6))
 (segment (start 168.55 106.45) (end 167.5 106.45) (width 0.5) (layer "B.Cu") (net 6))
 (segment (start 168.65 119.15) (end 167.5 119.15) (width 0.5) (layer "B.Cu") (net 6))
 (segment (start 173.75 88.81) (end 173.75 80.25) (width 0.5) (layer "B.Cu") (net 8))
 (segment (start 171.635 90.925) (end 173.75 88.81) (width 0.5) (layer "B.Cu") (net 8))
 (segment (start 157.52 80.25) (end 157.52 130.25) (width 0.5) (layer "B.Cu") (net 8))
 (segment (start 171.75 78.25) (end 158.5 78.25) (width 0.5) (layer "B.Cu") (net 8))
 (segment (start 173.75 80.25) (end 171.75 78.25) (width 0.5) (layer "B.Cu") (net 8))
 (segment (start 158.5 78.25) (end 157.52 79.23) (width 0.5) (layer "B.Cu") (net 8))
 (segment (start 157.52 79.23) (end 157.52 80.25) (width 0.5) (layer "B.Cu") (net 8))
 (segment (start 149.9 80.25) (end 149.9 130.25) (width 0.5) (layer "B.Cu") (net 5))
 (segment (start 146.235 85.845) (end 146.235 83.915) (width 0.5) (layer "B.Cu") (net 5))
 (segment (start 146.235 83.915) (end 149.9 80.25) (width 0.5) (layer "B.Cu") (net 5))
 (segment (start 158.23 77) (end 173.75 77) (width 0.5) (layer "B.Cu") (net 7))
 (segment (start 154.98 130.25) (end 154.98 80.25) (width 0.5) (layer "B.Cu") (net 7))
 (segment (start 176 94.18) (end 171.635 98.545) (width 0.5) (layer "B.Cu") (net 7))
 (segment (start 154.98 80.25) (end 158.23 77) (width 0.5) (layer "B.Cu") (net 7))
 (segment (start 176 79.25) (end 176 94.18) (width 0.5) (layer "B.Cu") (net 7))
 (segment (start 173.75 77) (end 176 79.25) (width 0.5) (layer "B.Cu") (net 7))
 (segment (start 175 122.23) (end 171.635 118.865) (width 0.5) (layer "B.Cu") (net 11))
 (segment (start 175 128.71) (end 175 122.23) (width 0.5) (layer "B.Cu") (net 11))
 (segment (start 162.6 130.25) (end 166.75 130.25) (width 0.5) (layer "B.Cu") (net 10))
 (segment (start 166.75 130.25) (end 167.5 129.5) (width 0.5) (layer "B.Cu") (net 10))
 (segment (start 167.5 129.5) (end 167.5 121.69) (width 0.5) (layer "B.Cu") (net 10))
 (segment (start 166.36 117.75) (end 167.5 116.61) (width 0.5) (layer "B.Cu") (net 19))
 (segment (start 162.6 117.75) (end 166.36 117.75) (width 0.5) (layer "B.Cu") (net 19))
 (segment (start 162.6 105.25) (end 162.6 110.6) (width 0.5) (layer "B.Cu") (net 15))
 (segment (start 163.53 111.53) (end 167.5 111.53) (width 0.5) (layer "B.Cu") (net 15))
 (segment (start 162.6 110.6) (end 163.53 111.53) (width 0.5) (layer "B.Cu") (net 15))
 (segment (start 162.6 99.01) (end 167.5 103.91) (width 0.5) (layer "B.Cu") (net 17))
 (segment (start 162.6 92.75) (end 162.6 99.01) (width 0.5) (layer "B.Cu") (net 17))
 (segment (start 164.5 82.15) (end 164.5 95.83) (width 0.5) (layer "B.Cu") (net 13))
 (segment (start 164.5 95.83) (end 167.5 98.83) (width 0.5) (layer "B.Cu") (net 13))
 (segment (start 162.6 80.25) (end 164.5 82.15) (width 0.5) (layer "B.Cu") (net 13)))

